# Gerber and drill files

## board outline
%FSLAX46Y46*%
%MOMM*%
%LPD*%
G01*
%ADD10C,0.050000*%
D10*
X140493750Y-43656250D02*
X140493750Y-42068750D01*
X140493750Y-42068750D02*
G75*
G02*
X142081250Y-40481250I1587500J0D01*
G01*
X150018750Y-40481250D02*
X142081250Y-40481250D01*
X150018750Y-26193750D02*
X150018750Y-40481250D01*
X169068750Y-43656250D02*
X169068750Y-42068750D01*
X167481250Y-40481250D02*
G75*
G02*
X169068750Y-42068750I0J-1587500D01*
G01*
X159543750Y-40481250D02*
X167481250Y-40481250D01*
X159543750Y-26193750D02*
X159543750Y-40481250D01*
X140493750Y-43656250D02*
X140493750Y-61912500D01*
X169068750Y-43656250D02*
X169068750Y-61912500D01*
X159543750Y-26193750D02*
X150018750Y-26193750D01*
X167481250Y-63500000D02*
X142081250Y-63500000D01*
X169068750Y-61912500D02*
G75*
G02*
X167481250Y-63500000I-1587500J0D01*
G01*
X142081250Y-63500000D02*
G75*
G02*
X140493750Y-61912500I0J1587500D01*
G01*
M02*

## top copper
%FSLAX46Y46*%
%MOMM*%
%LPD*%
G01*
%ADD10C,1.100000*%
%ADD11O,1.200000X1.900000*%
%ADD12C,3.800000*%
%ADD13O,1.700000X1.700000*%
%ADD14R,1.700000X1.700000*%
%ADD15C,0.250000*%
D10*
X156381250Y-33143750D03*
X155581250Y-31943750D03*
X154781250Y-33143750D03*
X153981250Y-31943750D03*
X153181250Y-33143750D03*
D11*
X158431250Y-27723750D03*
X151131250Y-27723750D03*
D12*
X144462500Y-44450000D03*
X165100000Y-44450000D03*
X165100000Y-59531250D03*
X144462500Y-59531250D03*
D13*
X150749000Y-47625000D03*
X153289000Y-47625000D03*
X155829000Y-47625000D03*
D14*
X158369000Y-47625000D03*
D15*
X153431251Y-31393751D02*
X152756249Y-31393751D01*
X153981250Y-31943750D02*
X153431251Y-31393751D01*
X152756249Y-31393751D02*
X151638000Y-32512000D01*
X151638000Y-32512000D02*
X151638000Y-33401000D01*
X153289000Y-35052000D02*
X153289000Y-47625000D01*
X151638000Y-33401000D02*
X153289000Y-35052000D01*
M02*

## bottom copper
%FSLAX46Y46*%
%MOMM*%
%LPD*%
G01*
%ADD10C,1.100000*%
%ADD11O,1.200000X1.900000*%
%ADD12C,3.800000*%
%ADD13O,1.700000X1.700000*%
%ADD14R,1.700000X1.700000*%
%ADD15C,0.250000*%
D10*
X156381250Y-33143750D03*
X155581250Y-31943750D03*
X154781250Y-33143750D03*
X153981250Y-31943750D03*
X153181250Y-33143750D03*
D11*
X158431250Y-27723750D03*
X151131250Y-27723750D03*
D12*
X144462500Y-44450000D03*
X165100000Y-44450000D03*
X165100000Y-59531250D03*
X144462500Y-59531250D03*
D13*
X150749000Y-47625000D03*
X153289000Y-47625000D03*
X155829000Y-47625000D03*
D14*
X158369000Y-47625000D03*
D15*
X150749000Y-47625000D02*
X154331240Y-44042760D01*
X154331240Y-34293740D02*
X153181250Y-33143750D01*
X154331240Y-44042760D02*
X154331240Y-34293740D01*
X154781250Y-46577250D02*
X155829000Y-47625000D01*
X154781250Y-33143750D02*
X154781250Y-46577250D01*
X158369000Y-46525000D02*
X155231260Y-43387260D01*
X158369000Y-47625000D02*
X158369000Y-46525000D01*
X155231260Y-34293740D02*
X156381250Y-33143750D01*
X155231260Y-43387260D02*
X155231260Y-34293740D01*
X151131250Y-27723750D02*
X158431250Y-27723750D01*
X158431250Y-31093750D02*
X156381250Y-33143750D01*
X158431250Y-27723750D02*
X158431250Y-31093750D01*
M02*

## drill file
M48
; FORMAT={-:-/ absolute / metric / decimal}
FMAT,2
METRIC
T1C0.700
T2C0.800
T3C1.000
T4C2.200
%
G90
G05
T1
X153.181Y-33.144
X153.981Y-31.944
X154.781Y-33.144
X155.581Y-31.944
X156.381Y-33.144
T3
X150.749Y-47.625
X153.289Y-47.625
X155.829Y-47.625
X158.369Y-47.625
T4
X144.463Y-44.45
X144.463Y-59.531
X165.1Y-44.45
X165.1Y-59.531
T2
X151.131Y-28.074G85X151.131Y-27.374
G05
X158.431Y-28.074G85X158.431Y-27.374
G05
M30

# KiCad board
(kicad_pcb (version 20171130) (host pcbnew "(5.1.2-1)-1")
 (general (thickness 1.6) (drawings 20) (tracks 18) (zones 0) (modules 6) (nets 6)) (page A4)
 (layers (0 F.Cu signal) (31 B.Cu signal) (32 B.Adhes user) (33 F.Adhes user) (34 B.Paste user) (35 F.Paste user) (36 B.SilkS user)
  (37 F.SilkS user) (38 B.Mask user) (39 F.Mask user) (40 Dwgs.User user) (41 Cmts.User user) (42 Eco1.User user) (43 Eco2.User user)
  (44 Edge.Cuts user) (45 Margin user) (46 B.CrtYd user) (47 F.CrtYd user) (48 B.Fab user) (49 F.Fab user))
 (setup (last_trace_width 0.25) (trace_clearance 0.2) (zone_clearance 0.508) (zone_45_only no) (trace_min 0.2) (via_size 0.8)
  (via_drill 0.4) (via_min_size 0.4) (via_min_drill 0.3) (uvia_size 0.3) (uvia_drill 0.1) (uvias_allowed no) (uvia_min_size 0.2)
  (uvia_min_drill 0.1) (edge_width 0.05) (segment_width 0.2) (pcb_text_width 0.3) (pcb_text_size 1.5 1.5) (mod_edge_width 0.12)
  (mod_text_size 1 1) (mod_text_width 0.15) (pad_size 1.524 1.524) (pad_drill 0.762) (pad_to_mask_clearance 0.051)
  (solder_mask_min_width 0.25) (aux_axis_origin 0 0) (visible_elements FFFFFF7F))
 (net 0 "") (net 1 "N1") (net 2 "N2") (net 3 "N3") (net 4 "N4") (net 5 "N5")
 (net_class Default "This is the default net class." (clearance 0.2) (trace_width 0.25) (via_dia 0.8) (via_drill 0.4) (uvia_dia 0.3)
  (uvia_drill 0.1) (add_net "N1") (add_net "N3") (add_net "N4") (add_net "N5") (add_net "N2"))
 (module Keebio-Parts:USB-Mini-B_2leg (layer F.Cu) (at 154.78125 32.54375 180)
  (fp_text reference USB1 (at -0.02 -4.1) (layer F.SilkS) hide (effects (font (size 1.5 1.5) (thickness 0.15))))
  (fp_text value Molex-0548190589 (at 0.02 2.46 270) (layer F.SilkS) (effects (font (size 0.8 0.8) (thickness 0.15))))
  (pad 1 thru_hole circle (at -1.6 -0.6 180) (size 1.1 1.1) (drill 0.7) (layers *.Cu *.Mask) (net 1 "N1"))
  (pad 2 thru_hole circle (at -0.8 0.6 180) (size 1.1 1.1) (drill 0.7) (layers *.Cu *.Mask) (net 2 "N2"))
  (pad 3 thru_hole circle (at 0 -0.6 180) (size 1.1 1.1) (drill 0.7) (layers *.Cu *.Mask) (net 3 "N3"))
  (pad 4 thru_hole circle (at 0.8 0.6 180) (size 1.1 1.1) (drill 0.7) (layers *.Cu *.Mask) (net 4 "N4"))
  (pad 5 thru_hole circle (at 1.6 -0.6 180) (size 1.1 1.1) (drill 0.7) (layers *.Cu *.Mask) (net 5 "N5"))
  (pad 6 thru_hole oval (at -3.65 4.82 180) (size 1.2 1.9) (drill oval 0.8 1.5) (layers *.Cu *.Mask) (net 1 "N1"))
  (pad 6 thru_hole oval (at 3.65 4.82 180) (size 1.2 1.9) (drill oval 0.8 1.5) (layers *.Cu *.Mask) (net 1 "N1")))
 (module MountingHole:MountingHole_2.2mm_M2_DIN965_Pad (layer F.Cu) (at 144.4625 44.45)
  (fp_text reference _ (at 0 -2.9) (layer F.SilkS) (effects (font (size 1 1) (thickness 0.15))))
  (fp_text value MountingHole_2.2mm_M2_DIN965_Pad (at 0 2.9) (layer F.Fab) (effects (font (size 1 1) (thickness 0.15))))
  (pad 1 thru_hole circle (at 0 0) (size 3.8 3.8) (drill 2.2) (layers *.Cu *.Mask)))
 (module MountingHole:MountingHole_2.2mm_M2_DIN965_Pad (layer F.Cu) (at 165.1 44.45)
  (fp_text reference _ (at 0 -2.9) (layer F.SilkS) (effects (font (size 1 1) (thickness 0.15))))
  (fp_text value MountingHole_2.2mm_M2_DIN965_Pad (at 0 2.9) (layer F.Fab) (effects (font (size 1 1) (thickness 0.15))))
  (pad 1 thru_hole circle (at 0 0) (size 3.8 3.8) (drill 2.2) (layers *.Cu *.Mask)))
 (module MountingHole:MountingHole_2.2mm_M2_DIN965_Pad (layer F.Cu) (at 165.1 59.53125)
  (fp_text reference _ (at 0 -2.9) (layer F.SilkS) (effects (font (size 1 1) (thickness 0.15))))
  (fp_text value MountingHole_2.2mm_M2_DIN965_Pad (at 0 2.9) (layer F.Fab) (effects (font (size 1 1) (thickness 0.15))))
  (pad 1 thru_hole circle (at 0 0) (size 3.8 3.8) (drill 2.2) (layers *.Cu *.Mask)))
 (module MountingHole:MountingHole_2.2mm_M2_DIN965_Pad (layer F.Cu) (at 144.4625 59.53125)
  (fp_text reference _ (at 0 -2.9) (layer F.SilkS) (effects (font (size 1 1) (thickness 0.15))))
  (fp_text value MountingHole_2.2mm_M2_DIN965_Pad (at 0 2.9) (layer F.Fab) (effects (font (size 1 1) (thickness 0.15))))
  (pad 1 thru_hole circle (at 0 0) (size 3.8 3.8) (drill 2.2) (layers *.Cu *.Mask)))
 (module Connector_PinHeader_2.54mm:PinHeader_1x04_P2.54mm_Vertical (layer F.Cu) (at 158.369 47.625 270)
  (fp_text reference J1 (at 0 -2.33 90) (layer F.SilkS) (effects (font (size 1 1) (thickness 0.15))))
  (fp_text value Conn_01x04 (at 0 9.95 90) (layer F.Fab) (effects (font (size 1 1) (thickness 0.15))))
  (pad 4 thru_hole oval (at 0 7.62 270) (size 1.7 1.7) (drill 1) (layers *.Cu *.Mask) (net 5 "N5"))
  (pad 3 thru_hole oval (at 0 5.08 270) (size 1.7 1.7) (drill 1) (layers *.Cu *.Mask) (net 4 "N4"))
  (pad 2 thru_hole oval (at 0 2.54 270) (size 1.7 1.7) (drill 1) (layers *.Cu *.Mask) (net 3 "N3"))
  (pad 1 thru_hole rect (at 0 0 270) (size 1.7 1.7) (drill 1) (layers *.Cu *.Mask) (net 1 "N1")))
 (gr_line (start 140.49375 43.65625) (end 140.49375 42.06875) (layer Edge.Cuts) (width 0.05))
 (gr_arc (start 142.08125 42.06875) (end 142.08125 40.48125) (angle -90) (layer Edge.Cuts) (width 0.05))
 (gr_line (start 150.01875 40.48125) (end 142.08125 40.48125) (layer Edge.Cuts) (width 0.05))
 (gr_line (start 150.01875 26.19375) (end 150.01875 40.48125) (layer Edge.Cuts) (width 0.05))
 (gr_line (start 169.06875 43.65625) (end 169.06875 42.06875) (layer Edge.Cuts) (width 0.05))
 (gr_arc (start 167.48125 42.06875) (end 169.06875 42.06875) (angle -90) (layer Edge.Cuts) (width 0.05))
 (gr_line (start 159.54375 40.48125) (end 167.48125 40.48125) (layer Edge.Cuts) (width 0.05))
 (gr_line (start 159.54375 26.19375) (end 159.54375 40.48125) (layer Edge.Cuts) (width 0.05))
 (gr_line (start 140.49375 43.65625) (end 140.49375 61.9125) (layer Edge.Cuts) (width 0.05))
 (gr_line (start 169.06875 43.65625) (end 169.06875 61.9125) (layer Edge.Cuts) (width 0.05))
 (gr_line (start 159.54375 26.19375) (end 150.01875 26.19375) (layer Edge.Cuts) (width 0.05))
 (gr_line (start 167.48125 63.5) (end 142.08125 63.5) (layer Edge.Cuts) (width 0.05))
 (gr_arc (start 167.48125 61.9125) (end 167.48125 63.5) (angle -90) (layer Edge.Cuts) (width 0.05))
 (gr_arc (start 142.08125 61.9125) (end 140.49375 61.9125) (angle -90) (layer Edge.Cuts) (width 0.05))
 (segment (start 150.749 47.625) (end 154.33124 44.04276) (width 0.25) (layer B.Cu) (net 5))
 (segment (start 154.33124 34.29374) (end 153.18125 33.14375) (width 0.25) (layer B.Cu) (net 5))
 (segment (start 154.33124 44.04276) (end 154.33124 34.29374) (width 0.25) (layer B.Cu) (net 5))
 (segment (start 153.431251 31.393751) (end 152.756249 31.393751) (width 0.25) (layer F.Cu) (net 4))
 (segment (start 153.98125 31.94375) (end 153.431251 31.393751) (width 0.25) (layer F.Cu) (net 4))
 (segment (start 152.756249 31.393751) (end 151.638 32.512) (width 0.25) (layer F.Cu) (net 4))
 (segment (start 151.638 32.512) (end 151.638 33.401) (width 0.25) (layer F.Cu) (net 4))
 (segment (start 153.289 35.052) (end 153.289 47.625) (width 0.25) (layer F.Cu) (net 4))
 (segment (start 151.638 33.401) (end 153.289 35.052) (width 0.25) (layer F.Cu) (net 4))
 (segment (start 154.78125 46.57725) (end 155.829 47.625) (width 0.25) (layer B.Cu) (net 3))
 (segment (start 154.78125 33.14375) (end 154.78125 46.57725) (width 0.25) (layer B.Cu) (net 3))
 (segment (start 158.369 46.525) (end 155.23126 43.38726) (width 0.25) (layer B.Cu) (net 1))
 (segment (start 158.369 47.625) (end 158.369 46.525) (width 0.25) (layer B.Cu) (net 1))
 (segment (start 155.23126 34.29374) (end 156.38125 33.14375) (width 0.25) (layer B.Cu) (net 1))
 (segment (start 155.23126 43.38726) (end 155.23126 34.29374) (width 0.25) (layer B.Cu) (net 1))
 (segment (start 151.13125 27.72375) (end 158.43125 27.72375) (width 0.25) (layer B.Cu) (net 1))
 (segment (start 158.43125 31.09375) (end 156.38125 33.14375) (width 0.25) (layer B.Cu) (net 1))
 (segment (start 158.43125 27.72375) (end 158.43125 31.09375) (width 0.25) (layer B.Cu) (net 1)))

